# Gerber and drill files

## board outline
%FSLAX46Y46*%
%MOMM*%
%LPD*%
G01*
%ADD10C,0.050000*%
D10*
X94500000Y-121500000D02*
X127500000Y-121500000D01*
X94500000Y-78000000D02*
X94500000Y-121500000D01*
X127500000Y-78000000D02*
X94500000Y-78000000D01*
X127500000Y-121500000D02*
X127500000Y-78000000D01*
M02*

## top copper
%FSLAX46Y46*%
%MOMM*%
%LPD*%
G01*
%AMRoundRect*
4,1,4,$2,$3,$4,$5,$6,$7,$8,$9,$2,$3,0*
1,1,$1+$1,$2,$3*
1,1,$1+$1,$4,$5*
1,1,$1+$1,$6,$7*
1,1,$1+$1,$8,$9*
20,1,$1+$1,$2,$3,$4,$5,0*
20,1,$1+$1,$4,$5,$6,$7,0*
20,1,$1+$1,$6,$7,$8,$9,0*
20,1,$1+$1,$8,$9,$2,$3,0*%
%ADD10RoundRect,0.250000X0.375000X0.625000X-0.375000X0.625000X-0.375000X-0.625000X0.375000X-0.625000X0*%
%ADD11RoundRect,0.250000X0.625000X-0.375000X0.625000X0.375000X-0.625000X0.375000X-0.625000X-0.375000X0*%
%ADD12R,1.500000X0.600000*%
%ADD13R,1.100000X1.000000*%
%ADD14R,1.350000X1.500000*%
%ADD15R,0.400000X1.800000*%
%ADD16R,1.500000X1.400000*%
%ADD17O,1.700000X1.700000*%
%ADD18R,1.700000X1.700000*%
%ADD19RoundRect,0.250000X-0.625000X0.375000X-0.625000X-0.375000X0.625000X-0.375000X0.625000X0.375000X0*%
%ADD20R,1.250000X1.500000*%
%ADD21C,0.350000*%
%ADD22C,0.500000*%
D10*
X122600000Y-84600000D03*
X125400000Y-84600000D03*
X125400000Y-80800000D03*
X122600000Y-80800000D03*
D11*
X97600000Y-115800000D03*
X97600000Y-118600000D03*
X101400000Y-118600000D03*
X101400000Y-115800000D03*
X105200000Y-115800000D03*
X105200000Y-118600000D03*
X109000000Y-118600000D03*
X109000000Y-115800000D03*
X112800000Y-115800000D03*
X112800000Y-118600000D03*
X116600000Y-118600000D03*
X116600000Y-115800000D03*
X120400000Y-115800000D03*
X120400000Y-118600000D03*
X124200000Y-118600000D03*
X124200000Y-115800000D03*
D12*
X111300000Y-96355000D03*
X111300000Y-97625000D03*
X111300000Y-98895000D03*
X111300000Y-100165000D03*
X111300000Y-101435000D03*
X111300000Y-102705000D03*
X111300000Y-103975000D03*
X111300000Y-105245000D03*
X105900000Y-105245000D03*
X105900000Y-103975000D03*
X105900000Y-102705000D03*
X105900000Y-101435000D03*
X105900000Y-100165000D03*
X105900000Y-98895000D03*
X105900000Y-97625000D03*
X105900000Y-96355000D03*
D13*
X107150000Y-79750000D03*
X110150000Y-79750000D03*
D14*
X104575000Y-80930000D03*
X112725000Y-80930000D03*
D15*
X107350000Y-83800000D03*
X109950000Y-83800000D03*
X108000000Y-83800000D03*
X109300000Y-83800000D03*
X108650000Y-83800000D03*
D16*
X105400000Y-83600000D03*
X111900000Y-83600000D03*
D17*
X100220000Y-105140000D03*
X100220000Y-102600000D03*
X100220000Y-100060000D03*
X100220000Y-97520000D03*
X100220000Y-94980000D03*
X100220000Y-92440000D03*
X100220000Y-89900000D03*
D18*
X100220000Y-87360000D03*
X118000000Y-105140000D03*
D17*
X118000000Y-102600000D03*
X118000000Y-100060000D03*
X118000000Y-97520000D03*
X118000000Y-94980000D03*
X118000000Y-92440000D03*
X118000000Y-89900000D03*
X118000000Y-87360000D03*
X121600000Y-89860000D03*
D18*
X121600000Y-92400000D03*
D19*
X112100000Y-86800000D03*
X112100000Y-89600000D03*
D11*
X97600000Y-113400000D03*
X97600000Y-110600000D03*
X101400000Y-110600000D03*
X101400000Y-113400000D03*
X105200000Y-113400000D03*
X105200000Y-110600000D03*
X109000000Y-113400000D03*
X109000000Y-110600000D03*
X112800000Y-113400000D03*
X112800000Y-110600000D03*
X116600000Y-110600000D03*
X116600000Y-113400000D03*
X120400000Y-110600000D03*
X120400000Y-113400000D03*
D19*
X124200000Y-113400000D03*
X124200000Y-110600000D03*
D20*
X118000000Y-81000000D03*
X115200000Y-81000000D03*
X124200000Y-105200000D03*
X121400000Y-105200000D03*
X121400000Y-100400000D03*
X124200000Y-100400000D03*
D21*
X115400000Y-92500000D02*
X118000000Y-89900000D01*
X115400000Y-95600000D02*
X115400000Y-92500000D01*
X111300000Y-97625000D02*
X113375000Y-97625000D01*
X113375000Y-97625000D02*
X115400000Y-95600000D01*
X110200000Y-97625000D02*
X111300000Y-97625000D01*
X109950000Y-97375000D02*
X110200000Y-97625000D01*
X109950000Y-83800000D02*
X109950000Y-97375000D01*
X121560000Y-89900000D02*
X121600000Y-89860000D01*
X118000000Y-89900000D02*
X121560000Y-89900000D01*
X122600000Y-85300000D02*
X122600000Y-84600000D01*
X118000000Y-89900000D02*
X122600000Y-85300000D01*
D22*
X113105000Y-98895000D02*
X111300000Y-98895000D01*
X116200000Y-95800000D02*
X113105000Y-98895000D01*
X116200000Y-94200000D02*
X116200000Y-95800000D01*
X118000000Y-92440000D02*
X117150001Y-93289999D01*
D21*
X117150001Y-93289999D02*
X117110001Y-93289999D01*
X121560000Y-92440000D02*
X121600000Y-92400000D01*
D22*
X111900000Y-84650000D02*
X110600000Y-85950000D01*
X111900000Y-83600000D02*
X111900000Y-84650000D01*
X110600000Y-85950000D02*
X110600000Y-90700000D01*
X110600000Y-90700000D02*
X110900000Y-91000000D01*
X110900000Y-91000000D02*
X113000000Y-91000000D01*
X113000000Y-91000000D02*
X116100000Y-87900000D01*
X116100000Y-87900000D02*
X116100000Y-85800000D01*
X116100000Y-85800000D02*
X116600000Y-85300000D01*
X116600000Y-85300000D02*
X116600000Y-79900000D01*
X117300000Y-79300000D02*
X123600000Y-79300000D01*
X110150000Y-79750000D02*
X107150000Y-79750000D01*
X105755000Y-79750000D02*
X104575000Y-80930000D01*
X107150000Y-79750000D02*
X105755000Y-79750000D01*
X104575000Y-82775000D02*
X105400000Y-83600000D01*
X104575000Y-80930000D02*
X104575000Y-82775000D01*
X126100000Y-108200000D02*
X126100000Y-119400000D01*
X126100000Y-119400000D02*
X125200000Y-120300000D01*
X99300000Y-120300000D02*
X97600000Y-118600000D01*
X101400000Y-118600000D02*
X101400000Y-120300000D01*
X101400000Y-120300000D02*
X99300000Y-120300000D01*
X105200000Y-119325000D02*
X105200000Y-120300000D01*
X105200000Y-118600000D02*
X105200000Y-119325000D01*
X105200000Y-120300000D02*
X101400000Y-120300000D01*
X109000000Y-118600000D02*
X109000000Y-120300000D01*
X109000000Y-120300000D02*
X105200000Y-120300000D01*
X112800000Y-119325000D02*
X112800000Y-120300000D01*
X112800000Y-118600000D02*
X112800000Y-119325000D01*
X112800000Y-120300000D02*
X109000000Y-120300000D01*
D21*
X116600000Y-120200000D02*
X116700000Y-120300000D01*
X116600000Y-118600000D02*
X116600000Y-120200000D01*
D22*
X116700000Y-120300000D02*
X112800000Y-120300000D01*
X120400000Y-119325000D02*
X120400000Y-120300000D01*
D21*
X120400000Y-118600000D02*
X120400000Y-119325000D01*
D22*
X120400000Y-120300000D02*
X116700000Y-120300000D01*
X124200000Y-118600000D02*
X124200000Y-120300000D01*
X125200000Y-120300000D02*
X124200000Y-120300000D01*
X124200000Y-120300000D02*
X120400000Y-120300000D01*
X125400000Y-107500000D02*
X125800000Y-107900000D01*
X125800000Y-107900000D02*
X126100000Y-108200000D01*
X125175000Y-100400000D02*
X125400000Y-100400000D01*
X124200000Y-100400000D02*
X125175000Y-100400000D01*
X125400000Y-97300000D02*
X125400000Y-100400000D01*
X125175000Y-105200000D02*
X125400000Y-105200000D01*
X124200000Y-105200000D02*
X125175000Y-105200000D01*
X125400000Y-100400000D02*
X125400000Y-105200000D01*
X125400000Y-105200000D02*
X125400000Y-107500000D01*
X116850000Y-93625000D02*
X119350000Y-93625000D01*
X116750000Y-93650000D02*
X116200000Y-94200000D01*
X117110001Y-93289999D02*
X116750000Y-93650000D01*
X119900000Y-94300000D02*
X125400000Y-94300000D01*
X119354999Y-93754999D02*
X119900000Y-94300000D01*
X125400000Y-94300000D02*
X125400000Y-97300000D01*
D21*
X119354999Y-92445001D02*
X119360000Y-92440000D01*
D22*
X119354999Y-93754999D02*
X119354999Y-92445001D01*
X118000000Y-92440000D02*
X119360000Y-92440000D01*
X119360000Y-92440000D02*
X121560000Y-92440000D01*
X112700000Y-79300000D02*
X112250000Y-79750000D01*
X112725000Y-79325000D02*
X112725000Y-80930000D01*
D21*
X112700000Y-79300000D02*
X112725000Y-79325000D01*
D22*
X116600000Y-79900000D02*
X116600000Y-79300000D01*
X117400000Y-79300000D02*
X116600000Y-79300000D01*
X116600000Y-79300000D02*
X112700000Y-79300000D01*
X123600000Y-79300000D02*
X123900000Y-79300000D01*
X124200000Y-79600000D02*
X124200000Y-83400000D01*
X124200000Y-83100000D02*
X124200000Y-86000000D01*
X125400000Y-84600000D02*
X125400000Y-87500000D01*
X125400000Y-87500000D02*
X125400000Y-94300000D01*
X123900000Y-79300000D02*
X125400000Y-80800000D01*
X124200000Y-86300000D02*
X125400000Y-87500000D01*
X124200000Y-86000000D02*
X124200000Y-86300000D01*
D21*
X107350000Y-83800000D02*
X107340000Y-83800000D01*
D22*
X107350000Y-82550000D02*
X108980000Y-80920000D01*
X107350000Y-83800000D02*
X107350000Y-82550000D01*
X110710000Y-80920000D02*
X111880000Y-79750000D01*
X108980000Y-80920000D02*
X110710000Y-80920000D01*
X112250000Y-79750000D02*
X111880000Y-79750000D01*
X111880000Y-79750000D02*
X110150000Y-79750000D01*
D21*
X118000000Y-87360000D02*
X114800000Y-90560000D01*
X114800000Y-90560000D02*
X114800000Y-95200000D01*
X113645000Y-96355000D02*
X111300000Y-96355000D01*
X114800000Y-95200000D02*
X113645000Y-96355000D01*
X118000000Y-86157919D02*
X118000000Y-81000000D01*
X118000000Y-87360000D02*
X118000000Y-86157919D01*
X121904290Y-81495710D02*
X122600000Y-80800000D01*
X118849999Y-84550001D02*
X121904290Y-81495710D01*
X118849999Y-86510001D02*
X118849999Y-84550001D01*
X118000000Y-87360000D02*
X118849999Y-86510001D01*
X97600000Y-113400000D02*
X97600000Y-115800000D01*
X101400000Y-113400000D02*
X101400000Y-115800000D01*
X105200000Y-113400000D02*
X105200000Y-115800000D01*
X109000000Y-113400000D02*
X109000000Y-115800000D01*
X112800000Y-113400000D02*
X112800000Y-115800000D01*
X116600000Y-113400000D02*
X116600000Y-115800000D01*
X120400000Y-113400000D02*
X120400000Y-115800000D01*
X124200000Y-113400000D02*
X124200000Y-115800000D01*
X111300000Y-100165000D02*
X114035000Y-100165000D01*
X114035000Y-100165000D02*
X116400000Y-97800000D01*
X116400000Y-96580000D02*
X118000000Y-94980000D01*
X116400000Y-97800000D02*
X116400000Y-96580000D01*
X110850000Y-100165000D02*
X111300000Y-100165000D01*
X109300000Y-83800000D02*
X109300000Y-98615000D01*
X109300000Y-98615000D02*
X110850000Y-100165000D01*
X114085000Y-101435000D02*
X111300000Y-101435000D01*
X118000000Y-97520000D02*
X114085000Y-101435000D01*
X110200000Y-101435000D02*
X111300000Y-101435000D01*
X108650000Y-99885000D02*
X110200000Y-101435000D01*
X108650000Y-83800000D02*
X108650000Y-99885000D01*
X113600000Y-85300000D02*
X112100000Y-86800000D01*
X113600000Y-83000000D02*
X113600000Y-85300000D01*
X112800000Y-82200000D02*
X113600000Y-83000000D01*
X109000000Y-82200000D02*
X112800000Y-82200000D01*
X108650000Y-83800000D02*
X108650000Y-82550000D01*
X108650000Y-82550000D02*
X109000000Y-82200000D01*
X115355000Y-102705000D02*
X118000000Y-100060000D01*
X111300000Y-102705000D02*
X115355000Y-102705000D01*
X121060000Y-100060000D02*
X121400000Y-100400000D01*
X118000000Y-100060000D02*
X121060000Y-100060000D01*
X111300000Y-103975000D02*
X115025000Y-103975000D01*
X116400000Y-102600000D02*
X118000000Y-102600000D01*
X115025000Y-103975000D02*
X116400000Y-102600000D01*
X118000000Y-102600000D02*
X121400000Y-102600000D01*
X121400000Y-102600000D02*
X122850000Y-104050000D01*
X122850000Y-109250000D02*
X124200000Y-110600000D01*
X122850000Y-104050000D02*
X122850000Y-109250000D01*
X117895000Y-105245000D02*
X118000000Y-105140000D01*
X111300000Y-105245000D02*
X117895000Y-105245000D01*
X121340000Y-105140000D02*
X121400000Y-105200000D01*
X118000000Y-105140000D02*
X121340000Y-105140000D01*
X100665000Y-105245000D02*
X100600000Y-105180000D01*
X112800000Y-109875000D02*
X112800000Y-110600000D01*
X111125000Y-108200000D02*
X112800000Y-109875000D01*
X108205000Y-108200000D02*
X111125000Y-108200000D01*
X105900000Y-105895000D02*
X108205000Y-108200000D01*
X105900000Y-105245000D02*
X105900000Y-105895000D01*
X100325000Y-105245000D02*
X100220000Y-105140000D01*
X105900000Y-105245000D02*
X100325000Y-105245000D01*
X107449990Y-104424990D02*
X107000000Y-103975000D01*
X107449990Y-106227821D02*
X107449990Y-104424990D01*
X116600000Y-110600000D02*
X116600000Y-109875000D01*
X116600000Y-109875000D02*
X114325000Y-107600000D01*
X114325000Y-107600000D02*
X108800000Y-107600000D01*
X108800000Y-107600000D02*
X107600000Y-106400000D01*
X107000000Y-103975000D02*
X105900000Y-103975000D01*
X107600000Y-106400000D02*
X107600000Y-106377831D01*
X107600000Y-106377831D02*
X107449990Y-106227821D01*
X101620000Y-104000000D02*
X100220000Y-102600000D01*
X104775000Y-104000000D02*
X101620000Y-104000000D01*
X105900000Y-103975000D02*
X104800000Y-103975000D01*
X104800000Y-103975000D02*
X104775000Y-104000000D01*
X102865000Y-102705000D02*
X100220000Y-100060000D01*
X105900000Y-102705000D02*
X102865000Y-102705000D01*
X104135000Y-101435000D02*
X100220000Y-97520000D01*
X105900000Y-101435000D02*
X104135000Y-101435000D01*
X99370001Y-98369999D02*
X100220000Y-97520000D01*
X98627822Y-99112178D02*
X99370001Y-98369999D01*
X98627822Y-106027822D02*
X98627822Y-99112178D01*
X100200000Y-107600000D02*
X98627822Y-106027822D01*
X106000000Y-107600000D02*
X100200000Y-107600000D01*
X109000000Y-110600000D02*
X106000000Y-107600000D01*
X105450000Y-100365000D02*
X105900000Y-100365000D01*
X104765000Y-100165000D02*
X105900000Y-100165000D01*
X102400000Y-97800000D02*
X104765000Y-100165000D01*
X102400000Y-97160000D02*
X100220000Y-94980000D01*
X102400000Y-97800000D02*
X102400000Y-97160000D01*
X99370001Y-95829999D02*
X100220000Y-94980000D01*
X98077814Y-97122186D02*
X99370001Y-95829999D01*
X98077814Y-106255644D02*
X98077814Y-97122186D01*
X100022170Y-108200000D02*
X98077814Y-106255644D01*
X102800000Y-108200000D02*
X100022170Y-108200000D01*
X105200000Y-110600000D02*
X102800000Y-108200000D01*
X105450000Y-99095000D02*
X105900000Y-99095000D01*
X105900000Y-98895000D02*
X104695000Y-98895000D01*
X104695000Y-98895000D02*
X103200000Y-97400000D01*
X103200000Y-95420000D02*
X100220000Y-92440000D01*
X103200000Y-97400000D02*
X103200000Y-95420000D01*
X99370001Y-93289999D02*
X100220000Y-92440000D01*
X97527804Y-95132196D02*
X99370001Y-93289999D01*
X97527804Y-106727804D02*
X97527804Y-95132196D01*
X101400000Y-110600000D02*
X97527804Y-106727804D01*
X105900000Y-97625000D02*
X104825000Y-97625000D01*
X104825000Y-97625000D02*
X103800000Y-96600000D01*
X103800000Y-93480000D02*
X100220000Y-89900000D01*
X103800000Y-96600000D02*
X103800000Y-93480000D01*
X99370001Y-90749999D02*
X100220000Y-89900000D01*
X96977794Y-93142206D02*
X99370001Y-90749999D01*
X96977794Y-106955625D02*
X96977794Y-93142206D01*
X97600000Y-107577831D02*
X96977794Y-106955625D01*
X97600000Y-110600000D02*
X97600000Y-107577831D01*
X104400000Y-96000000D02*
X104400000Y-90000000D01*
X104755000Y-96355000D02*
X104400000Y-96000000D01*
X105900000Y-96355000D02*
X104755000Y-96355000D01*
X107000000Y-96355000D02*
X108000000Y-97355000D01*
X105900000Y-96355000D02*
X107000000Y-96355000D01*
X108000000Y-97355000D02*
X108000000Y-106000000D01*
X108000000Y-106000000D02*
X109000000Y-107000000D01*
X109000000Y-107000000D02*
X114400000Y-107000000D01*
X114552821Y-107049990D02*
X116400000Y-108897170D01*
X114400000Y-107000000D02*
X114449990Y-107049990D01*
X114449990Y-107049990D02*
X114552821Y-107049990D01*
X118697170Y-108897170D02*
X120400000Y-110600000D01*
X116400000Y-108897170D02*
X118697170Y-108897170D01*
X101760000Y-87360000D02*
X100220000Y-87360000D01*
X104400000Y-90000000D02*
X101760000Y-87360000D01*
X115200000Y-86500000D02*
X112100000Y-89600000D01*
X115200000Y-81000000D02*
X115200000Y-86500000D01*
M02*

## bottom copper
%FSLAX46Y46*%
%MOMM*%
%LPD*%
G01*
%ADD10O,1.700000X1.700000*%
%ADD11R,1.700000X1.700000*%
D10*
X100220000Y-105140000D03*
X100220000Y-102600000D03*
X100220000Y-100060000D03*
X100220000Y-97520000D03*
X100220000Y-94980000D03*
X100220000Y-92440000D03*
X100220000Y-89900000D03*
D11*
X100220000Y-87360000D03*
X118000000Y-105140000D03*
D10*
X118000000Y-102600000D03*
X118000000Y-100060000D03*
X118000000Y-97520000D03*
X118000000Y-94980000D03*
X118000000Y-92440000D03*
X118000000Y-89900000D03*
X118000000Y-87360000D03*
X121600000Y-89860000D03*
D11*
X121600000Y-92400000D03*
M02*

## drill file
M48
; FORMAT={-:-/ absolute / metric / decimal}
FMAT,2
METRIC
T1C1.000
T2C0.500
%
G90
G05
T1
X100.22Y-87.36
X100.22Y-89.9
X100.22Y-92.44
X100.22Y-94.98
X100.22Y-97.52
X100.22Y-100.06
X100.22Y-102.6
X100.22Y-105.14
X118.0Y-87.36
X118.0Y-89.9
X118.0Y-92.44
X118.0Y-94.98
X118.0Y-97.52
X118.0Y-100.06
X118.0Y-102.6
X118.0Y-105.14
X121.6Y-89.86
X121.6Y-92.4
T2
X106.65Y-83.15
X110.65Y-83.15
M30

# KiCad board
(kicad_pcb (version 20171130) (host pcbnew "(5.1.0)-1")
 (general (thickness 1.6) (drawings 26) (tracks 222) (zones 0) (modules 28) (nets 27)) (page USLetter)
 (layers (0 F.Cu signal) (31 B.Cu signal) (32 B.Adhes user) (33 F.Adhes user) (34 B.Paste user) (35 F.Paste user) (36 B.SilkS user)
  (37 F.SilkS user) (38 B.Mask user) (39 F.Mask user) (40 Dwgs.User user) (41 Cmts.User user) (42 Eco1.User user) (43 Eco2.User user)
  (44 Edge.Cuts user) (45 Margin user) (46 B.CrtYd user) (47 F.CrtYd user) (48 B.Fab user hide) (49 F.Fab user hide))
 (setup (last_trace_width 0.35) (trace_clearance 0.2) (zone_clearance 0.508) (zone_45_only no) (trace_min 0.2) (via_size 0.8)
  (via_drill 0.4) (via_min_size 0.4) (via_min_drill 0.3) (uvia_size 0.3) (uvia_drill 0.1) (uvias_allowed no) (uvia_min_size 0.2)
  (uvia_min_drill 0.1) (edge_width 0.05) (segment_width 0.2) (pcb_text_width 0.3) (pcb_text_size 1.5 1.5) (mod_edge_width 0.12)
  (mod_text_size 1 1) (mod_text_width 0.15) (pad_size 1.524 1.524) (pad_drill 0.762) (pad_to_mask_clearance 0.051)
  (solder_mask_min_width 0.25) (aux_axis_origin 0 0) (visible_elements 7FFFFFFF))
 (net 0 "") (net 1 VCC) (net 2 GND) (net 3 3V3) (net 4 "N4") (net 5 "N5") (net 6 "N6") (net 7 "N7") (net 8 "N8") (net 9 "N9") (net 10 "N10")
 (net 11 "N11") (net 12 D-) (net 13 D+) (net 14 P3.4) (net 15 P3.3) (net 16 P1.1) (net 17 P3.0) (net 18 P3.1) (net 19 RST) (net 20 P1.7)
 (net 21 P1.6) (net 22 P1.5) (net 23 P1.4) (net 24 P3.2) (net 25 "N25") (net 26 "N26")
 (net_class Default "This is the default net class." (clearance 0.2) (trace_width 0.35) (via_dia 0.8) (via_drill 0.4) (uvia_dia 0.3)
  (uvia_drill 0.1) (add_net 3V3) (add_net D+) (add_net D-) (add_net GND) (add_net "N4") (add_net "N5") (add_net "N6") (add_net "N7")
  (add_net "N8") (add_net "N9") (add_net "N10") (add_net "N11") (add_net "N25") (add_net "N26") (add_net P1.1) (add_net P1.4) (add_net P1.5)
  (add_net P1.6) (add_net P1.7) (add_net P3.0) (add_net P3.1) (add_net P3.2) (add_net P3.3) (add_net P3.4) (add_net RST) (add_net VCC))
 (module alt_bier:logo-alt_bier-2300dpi (layer F.Cu) (at 106.36 90.52)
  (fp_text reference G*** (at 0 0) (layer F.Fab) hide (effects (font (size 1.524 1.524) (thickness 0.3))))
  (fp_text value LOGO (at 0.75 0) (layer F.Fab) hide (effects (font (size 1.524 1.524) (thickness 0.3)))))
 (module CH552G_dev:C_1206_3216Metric (layer F.Cu) (at 124 84.6 180)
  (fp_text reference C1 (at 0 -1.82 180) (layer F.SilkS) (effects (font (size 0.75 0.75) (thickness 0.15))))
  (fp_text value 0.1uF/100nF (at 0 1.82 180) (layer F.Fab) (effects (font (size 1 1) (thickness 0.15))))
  (pad 2 smd roundrect (at 1.4 0 180) (size 1.25 1.75) (layers F.Cu F.Paste F.Mask) (roundrect_rratio 0.2) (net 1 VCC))
  (pad 1 smd roundrect (at -1.4 0 180) (size 1.25 1.75) (layers F.Cu F.Paste F.Mask) (roundrect_rratio 0.2) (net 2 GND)))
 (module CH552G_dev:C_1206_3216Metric (layer F.Cu) (at 124 80.8 180)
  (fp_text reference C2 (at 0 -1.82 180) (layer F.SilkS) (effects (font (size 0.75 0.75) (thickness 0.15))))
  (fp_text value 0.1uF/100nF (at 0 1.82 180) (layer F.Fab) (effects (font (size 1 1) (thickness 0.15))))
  (pad 1 smd roundrect (at -1.4 0 180) (size 1.25 1.75) (layers F.Cu F.Paste F.Mask) (roundrect_rratio 0.2) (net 2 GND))
  (pad 2 smd roundrect (at 1.4 0 180) (size 1.25 1.75) (layers F.Cu F.Paste F.Mask) (roundrect_rratio 0.2) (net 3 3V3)))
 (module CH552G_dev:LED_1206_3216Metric (layer F.Cu) (at 97.6 117.2 90)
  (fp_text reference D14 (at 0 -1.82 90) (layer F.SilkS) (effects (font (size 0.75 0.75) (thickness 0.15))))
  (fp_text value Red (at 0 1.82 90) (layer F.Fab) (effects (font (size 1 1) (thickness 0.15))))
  (pad 2 smd roundrect (at 1.4 0 90) (size 1.25 1.75) (layers F.Cu F.Paste F.Mask) (roundrect_rratio 0.2) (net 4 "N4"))
  (pad 1 smd roundrect (at -1.4 0 90) (size 1.25 1.75) (layers F.Cu F.Paste F.Mask) (roundrect_rratio 0.2) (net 2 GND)))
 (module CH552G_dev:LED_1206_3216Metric (layer F.Cu) (at 101.4 117.2 90)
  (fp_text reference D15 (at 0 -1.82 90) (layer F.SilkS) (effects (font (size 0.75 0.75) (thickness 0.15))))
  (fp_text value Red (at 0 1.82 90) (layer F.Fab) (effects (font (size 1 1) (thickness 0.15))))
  (pad 1 smd roundrect (at -1.4 0 90) (size 1.25 1.75) (layers F.Cu F.Paste F.Mask) (roundrect_rratio 0.2) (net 2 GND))
  (pad 2 smd roundrect (at 1.4 0 90) (size 1.25 1.75) (layers F.Cu F.Paste F.Mask) (roundrect_rratio 0.2) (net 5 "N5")))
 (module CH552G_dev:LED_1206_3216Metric (layer F.Cu) (at 105.2 117.2 90)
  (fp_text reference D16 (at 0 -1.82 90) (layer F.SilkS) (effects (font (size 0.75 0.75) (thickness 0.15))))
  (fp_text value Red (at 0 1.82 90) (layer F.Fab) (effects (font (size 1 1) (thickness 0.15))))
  (pad 2 smd roundrect (at 1.4 0 90) (size 1.25 1.75) (layers F.Cu F.Paste F.Mask) (roundrect_rratio 0.2) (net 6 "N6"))
  (pad 1 smd roundrect (at -1.4 0 90) (size 1.25 1.75) (layers F.Cu F.Paste F.Mask) (roundrect_rratio 0.2) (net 2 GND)))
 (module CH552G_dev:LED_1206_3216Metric (layer F.Cu) (at 109 117.2 90)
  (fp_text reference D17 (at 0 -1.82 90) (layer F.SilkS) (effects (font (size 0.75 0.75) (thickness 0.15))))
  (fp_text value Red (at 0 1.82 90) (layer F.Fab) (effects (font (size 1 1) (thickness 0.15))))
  (pad 1 smd roundrect (at -1.4 0 90) (size 1.25 1.75) (layers F.Cu F.Paste F.Mask) (roundrect_rratio 0.2) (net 2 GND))
  (pad 2 smd roundrect (at 1.4 0 90) (size 1.25 1.75) (layers F.Cu F.Paste F.Mask) (roundrect_rratio 0.2) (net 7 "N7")))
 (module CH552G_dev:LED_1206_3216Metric (layer F.Cu) (at 112.8 117.2 90)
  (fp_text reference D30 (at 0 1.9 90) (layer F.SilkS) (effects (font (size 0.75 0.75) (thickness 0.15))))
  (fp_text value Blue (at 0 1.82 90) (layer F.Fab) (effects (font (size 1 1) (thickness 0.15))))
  (pad 2 smd roundrect (at 1.4 0 90) (size 1.25 1.75) (layers F.Cu F.Paste F.Mask) (roundrect_rratio 0.2) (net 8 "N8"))
  (pad 1 smd roundrect (at -1.4 0 90) (size 1.25 1.75) (layers F.Cu F.Paste F.Mask) (roundrect_rratio 0.2) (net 2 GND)))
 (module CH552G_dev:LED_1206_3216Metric (layer F.Cu) (at 116.6 117.2 90)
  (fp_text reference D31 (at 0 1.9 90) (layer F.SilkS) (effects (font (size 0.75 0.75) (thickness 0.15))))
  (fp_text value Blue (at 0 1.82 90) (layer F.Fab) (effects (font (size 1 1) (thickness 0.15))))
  (pad 1 smd roundrect (at -1.4 0 90) (size 1.25 1.75) (layers F.Cu F.Paste F.Mask) (roundrect_rratio 0.2) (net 2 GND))
  (pad 2 smd roundrect (at 1.4 0 90) (size 1.25 1.75) (layers F.Cu F.Paste F.Mask) (roundrect_rratio 0.2) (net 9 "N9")))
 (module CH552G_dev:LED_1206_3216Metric (layer F.Cu) (at 120.4 117.2 90)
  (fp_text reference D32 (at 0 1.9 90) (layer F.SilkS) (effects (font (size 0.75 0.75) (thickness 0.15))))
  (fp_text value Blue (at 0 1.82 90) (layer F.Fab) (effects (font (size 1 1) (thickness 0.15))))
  (pad 2 smd roundrect (at 1.4 0 90) (size 1.25 1.75) (layers F.Cu F.Paste F.Mask) (roundrect_rratio 0.2) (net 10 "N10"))
  (pad 1 smd roundrect (at -1.4 0 90) (size 1.25 1.75) (layers F.Cu F.Paste F.Mask) (roundrect_rratio 0.2) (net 2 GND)))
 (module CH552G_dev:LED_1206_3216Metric (layer F.Cu) (at 124.2 117.2 90)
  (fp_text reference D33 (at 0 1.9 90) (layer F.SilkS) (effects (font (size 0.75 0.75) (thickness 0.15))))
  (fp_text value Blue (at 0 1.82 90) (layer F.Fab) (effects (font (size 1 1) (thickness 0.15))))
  (pad 1 smd roundrect (at -1.4 0 90) (size 1.25 1.75) (layers F.Cu F.Paste F.Mask) (roundrect_rratio 0.2) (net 2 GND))
  (pad 2 smd roundrect (at 1.4 0 90) (size 1.25 1.75) (layers F.Cu F.Paste F.Mask) (roundrect_rratio 0.2) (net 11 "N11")))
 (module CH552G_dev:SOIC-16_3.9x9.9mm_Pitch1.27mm (layer F.Cu) (at 108.6 100.8)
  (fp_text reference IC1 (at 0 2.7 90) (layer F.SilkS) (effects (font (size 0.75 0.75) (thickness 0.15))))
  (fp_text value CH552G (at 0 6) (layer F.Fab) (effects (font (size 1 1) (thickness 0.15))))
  (pad 16 smd rect (at 2.7 -4.445) (size 1.5 0.6) (layers F.Cu F.Paste F.Mask) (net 3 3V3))
  (pad 15 smd rect (at 2.7 -3.175) (size 1.5 0.6) (layers F.Cu F.Paste F.Mask) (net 1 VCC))
  (pad 14 smd rect (at 2.7 -1.905) (size 1.5 0.6) (layers F.Cu F.Paste F.Mask) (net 2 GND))
  (pad 13 smd rect (at 2.7 -0.635) (size 1.5 0.6) (layers F.Cu F.Paste F.Mask) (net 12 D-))
  (pad 12 smd rect (at 2.7 0.635) (size 1.5 0.6) (layers F.Cu F.Paste F.Mask) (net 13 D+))
  (pad 11 smd rect (at 2.7 1.905) (size 1.5 0.6) (layers F.Cu F.Paste F.Mask) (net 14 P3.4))
  (pad 10 smd rect (at 2.7 3.175) (size 1.5 0.6) (layers F.Cu F.Paste F.Mask) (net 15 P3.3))
  (pad 9 smd rect (at 2.7 4.445) (size 1.5 0.6) (layers F.Cu F.Paste F.Mask) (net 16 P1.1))
  (pad 8 smd rect (at -2.7 4.445) (size 1.5 0.6) (layers F.Cu F.Paste F.Mask) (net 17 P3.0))
  (pad 7 smd rect (at -2.7 3.175) (size 1.5 0.6) (layers F.Cu F.Paste F.Mask) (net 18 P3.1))
  (pad 6 smd rect (at -2.7 1.905) (size 1.5 0.6) (layers F.Cu F.Paste F.Mask) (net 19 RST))
  (pad 5 smd rect (at -2.7 0.635) (size 1.5 0.6) (layers F.Cu F.Paste F.Mask) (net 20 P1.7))
  (pad 4 smd rect (at -2.7 -0.635) (size 1.5 0.6) (layers F.Cu F.Paste F.Mask) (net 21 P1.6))
  (pad 3 smd rect (at -2.7 -1.905) (size 1.5 0.6) (layers F.Cu F.Paste F.Mask) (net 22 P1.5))
  (pad 2 smd rect (at -2.7 -3.175) (size 1.5 0.6) (layers F.Cu F.Paste F.Mask) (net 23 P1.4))
  (pad 1 smd rect (at -2.7 -4.445) (size 1.5 0.6) (layers F.Cu F.Paste F.Mask) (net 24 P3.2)))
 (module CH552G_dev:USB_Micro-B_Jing (layer F.Cu) (at 108.65 81.7 180)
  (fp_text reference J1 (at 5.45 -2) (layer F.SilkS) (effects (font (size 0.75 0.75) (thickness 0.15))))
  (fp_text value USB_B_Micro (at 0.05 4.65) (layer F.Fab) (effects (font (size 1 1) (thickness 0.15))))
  (pad 6 smd rect (at 1.5 1.95 180) (size 1.1 1) (layers F.Cu F.Paste F.Mask) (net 2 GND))
  (pad 6 smd rect (at -1.5 1.95 180) (size 1.1 1) (layers F.Cu F.Paste F.Mask) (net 2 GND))
  (pad 6 smd rect (at 4.075 0.77 180) (size 1.35 1.5) (layers F.Cu F.Paste F.Mask) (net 2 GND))
  (pad 6 smd rect (at -4.075 0.77 180) (size 1.35 1.5) (layers F.Cu F.Paste F.Mask) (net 2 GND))
  (pad "" np_thru_hole circle (at 2 -1.45 180) (size 0.5 0.5) (drill 0.5) (layers *.Cu *.Mask))
  (pad "" np_thru_hole circle (at -2 -1.45 180) (size 0.5 0.5) (drill 0.5) (layers *.Cu *.Mask))
  (pad 5 smd rect (at 1.3 -2.1 180) (size 0.4 1.8) (layers F.Cu F.Paste F.Mask) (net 2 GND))
  (pad 1 smd rect (at -1.3 -2.1 180) (size 0.4 1.8) (layers F.Cu F.Paste F.Mask) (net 1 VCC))
  (pad 4 smd rect (at 0.65 -2.1 180) (size 0.4 1.8) (layers F.Cu F.Paste F.Mask) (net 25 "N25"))
  (pad 2 smd rect (at -0.65 -2.1 180) (size 0.4 1.8) (layers F.Cu F.Paste F.Mask) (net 12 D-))
  (pad 3 smd rect (at 0 -2.1 180) (size 0.4 1.8) (layers F.Cu F.Paste F.Mask) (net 13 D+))
  (pad 6 smd rect (at 3.25 -1.9 180) (size 1.5 1.4) (layers F.Cu F.Paste F.Mask) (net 2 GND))
  (pad 6 smd rect (at -3.25 -1.9 180) (size 1.5 1.4) (layers F.Cu F.Paste F.Mask) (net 2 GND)))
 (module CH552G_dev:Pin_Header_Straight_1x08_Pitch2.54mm (layer F.Cu) (at 100.22 87.36)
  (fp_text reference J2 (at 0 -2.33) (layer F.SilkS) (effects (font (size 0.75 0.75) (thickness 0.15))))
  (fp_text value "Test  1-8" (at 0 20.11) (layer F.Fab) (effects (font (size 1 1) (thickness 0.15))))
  (pad 8 thru_hole oval (at 0 17.78) (size 1.7 1.7) (drill 1) (layers *.Cu *.Mask) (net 17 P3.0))
  (pad 7 thru_hole oval (at 0 15.24) (size 1.7 1.7) (drill 1) (layers *.Cu *.Mask) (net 18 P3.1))
  (pad 6 thru_hole oval (at 0 12.7) (size 1.7 1.7) (drill 1) (layers *.Cu *.Mask) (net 19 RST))
  (pad 5 thru_hole oval (at 0 10.16) (size 1.7 1.7) (drill 1) (layers *.Cu *.Mask) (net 20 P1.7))
  (pad 4 thru_hole oval (at 0 7.62) (size 1.7 1.7) (drill 1) (layers *.Cu *.Mask) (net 21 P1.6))
  (pad 3 thru_hole oval (at 0 5.08) (size 1.7 1.7) (drill 1) (layers *.Cu *.Mask) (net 22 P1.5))
  (pad 2 thru_hole oval (at 0 2.54) (size 1.7 1.7) (drill 1) (layers *.Cu *.Mask) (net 23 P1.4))
  (pad 1 thru_hole rect (at 0 0) (size 1.7 1.7) (drill 1) (layers *.Cu *.Mask) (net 24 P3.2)))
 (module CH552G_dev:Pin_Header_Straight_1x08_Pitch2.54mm (layer F.Cu) (at 118 105.14 180)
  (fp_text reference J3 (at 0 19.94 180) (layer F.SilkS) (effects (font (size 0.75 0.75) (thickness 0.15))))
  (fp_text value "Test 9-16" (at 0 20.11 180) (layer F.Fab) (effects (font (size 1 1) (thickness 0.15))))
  (pad 1 thru_hole rect (at 0 0 180) (size 1.7 1.7) (drill 1) (layers *.Cu *.Mask) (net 16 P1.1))
  (pad 2 thru_hole oval (at 0 2.54 180) (size 1.7 1.7) (drill 1) (layers *.Cu *.Mask) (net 15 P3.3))
  (pad 3 thru_hole oval (at 0 5.08 180) (size 1.7 1.7) (drill 1) (layers *.Cu *.Mask) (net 14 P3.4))
  (pad 4 thru_hole oval (at 0 7.62 180) (size 1.7 1.7) (drill 1) (layers *.Cu *.Mask) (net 13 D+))
  (pad 5 thru_hole oval (at 0 10.16 180) (size 1.7 1.7) (drill 1) (layers *.Cu *.Mask) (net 12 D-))
  (pad 6 thru_hole oval (at 0 12.7 180) (size 1.7 1.7) (drill 1) (layers *.Cu *.Mask) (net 2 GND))
  (pad 7 thru_hole oval (at 0 15.24 180) (size 1.7 1.7) (drill 1) (layers *.Cu *.Mask) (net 1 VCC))
  (pad 8 thru_hole oval (at 0 17.78 180) (size 1.7 1.7) (drill 1) (layers *.Cu *.Mask) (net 3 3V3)))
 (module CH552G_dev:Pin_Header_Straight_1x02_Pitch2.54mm (layer F.Cu) (at 121.6 92.4 180)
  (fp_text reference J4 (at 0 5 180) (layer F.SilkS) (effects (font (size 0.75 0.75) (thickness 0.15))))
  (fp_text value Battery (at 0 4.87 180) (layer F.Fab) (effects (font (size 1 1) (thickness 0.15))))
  (pad 2 thru_hole oval (at 0 2.54 180) (size 1.7 1.7) (drill 1) (layers *.Cu *.Mask) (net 1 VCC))
  (pad 1 thru_hole rect (at 0 0 180) (size 1.7 1.7) (drill 1) (layers *.Cu *.Mask) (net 2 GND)))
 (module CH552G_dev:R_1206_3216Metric (layer F.Cu) (at 112.1 88.2 270)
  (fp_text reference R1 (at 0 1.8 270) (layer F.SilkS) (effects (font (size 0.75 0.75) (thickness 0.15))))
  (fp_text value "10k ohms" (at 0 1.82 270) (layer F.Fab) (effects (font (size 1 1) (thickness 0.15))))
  (pad 1 smd roundrect (at -1.4 0 270) (size 1.25 1.75) (layers F.Cu F.Paste F.Mask) (roundrect_rratio 0.2) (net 13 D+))
  (pad 2 smd roundrect (at 1.4 0 270) (size 1.25 1.75) (layers F.Cu F.Paste F.Mask) (roundrect_rratio 0.2) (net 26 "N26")))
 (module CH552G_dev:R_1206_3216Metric (layer F.Cu) (at 97.6 112 90)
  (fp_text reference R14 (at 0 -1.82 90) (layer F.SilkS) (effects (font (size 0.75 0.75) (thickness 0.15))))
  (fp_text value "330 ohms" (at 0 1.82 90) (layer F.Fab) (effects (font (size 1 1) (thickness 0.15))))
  (pad 1 smd roundrect (at -1.4 0 90) (size 1.25 1.75) (layers F.Cu F.Paste F.Mask) (roundrect_rratio 0.2) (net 4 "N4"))
  (pad 2 smd roundrect (at 1.4 0 90) (size 1.25 1.75) (layers F.Cu F.Paste F.Mask) (roundrect_rratio 0.2) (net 23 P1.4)))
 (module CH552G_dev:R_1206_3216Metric (layer F.Cu) (at 101.4 112 90)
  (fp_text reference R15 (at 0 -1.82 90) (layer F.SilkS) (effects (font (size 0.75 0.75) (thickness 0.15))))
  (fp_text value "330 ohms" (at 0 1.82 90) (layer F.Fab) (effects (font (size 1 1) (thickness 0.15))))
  (pad 2 smd roundrect (at 1.4 0 90) (size 1.25 1.75) (layers F.Cu F.Paste F.Mask) (roundrect_rratio 0.2) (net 22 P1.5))
  (pad 1 smd roundrect (at -1.4 0 90) (size 1.25 1.75) (layers F.Cu F.Paste F.Mask) (roundrect_rratio 0.2) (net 5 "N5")))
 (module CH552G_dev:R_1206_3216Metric (layer F.Cu) (at 105.2 112 90)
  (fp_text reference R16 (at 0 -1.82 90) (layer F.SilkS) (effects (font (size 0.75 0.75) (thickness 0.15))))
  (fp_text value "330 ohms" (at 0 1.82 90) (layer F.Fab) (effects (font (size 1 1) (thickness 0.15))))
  (pad 1 smd roundrect (at -1.4 0 90) (size 1.25 1.75) (layers F.Cu F.Paste F.Mask) (roundrect_rratio 0.2) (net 6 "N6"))
  (pad 2 smd roundrect (at 1.4 0 90) (size 1.25 1.75) (layers F.Cu F.Paste F.Mask) (roundrect_rratio 0.2) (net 21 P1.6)))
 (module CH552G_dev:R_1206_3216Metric (layer F.Cu) (at 109 112 90)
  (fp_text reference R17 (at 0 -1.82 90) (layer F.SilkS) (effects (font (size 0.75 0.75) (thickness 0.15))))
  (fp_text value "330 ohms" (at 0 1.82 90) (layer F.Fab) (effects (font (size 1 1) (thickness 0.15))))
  (pad 1 smd roundrect (at -1.4 0 90) (size 1.25 1.75) (layers F.Cu F.Paste F.Mask) (roundrect_rratio 0.2) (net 7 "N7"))
  (pad 2 smd roundrect (at 1.4 0 90) (size 1.25 1.75) (layers F.Cu F.Paste F.Mask) (roundrect_rratio 0.2) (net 20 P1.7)))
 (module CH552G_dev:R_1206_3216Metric (layer F.Cu) (at 112.8 112 90)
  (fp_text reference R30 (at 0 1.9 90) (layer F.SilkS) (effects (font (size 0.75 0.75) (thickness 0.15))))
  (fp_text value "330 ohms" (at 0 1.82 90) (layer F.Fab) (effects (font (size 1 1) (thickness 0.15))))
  (pad 1 smd roundrect (at -1.4 0 90) (size 1.25 1.75) (layers F.Cu F.Paste F.Mask) (roundrect_rratio 0.2) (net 8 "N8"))
  (pad 2 smd roundrect (at 1.4 0 90) (size 1.25 1.75) (layers F.Cu F.Paste F.Mask) (roundrect_rratio 0.2) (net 17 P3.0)))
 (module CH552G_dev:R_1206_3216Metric (layer F.Cu) (at 116.6 112 90)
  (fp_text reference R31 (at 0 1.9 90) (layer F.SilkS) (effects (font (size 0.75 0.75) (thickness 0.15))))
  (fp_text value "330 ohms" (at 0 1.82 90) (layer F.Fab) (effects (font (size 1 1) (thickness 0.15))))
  (pad 2 smd roundrect (at 1.4 0 90) (size 1.25 1.75) (layers F.Cu F.Paste F.Mask) (roundrect_rratio 0.2) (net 18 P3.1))
  (pad 1 smd roundrect (at -1.4 0 90) (size 1.25 1.75) (layers F.Cu F.Paste F.Mask) (roundrect_rratio 0.2) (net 9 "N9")))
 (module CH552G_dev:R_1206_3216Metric (layer F.Cu) (at 120.4 112 90)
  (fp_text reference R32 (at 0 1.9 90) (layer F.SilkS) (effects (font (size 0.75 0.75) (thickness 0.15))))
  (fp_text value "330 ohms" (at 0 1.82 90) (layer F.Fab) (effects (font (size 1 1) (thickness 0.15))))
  (pad 2 smd roundrect (at 1.4 0 90) (size 1.25 1.75) (layers F.Cu F.Paste F.Mask) (roundrect_rratio 0.2) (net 24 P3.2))
  (pad 1 smd roundrect (at -1.4 0 90) (size 1.25 1.75) (layers F.Cu F.Paste F.Mask) (roundrect_rratio 0.2) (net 10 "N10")))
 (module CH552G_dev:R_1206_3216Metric (layer F.Cu) (at 124.2 112 270)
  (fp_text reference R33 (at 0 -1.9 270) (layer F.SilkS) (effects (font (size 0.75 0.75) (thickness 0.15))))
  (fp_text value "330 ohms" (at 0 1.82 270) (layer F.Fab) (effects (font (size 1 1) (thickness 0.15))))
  (pad 2 smd roundrect (at 1.4 0 270) (size 1.25 1.75) (layers F.Cu F.Paste F.Mask) (roundrect_rratio 0.2) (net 11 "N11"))
  (pad 1 smd roundrect (at -1.4 0 270) (size 1.25 1.75) (layers F.Cu F.Paste F.Mask) (roundrect_rratio 0.2) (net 15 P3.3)))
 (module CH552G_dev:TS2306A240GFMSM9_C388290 (layer F.Cu) (at 116.6 81 180)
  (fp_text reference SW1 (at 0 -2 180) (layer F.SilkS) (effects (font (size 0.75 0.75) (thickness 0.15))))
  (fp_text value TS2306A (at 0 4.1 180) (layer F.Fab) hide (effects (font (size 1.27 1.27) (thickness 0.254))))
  (pad 1 smd rect (at -1.4 0 180) (size 1.25 1.5) (layers F.Cu F.Paste F.Mask) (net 3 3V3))
  (pad 2 smd rect (at 1.4 0 180) (size 1.25 1.5) (layers F.Cu F.Paste F.Mask) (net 26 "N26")))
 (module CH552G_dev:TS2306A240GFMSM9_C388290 (layer F.Cu) (at 122.8 105.2)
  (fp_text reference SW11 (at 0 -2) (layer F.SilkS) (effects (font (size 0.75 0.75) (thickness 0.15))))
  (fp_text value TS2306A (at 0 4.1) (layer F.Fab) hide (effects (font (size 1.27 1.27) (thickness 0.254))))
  (pad 2 smd rect (at 1.4 0) (size 1.25 1.5) (layers F.Cu F.Paste F.Mask) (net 2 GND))
  (pad 1 smd rect (at -1.4 0) (size 1.25 1.5) (layers F.Cu F.Paste F.Mask) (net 16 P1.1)))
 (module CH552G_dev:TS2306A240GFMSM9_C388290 (layer F.Cu) (at 122.8 100.4)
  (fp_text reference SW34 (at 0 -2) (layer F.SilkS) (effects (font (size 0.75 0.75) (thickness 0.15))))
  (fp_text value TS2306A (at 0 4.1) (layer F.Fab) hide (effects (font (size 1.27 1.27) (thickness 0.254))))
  (pad 1 smd rect (at -1.4 0) (size 1.25 1.5) (layers F.Cu F.Paste F.Mask) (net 14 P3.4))
  (pad 2 smd rect (at 1.4 0) (size 1.25 1.5) (layers F.Cu F.Paste F.Mask) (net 2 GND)))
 (gr_line (start 94.5 121.5) (end 127.5 121.5) (layer Edge.Cuts) (width 0.05))
 (gr_line (start 94.5 78) (end 94.5 121.5) (layer Edge.Cuts) (width 0.05))
 (gr_line (start 127.5 78) (end 94.5 78) (layer Edge.Cuts) (width 0.05))
 (gr_line (start 127.5 121.5) (end 127.5 78) (layer Edge.Cuts) (width 0.05))
 (segment (start 115.4 92.5) (end 118 89.9) (width 0.35) (layer F.Cu) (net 1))
 (segment (start 115.4 95.6) (end 115.4 92.5) (width 0.35) (layer F.Cu) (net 1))
 (segment (start 111.3 97.625) (end 113.375 97.625) (width 0.35) (layer F.Cu) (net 1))
 (segment (start 113.375 97.625) (end 115.4 95.6) (width 0.35) (layer F.Cu) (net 1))
 (segment (start 110.2 97.625) (end 111.3 97.625) (width 0.35) (layer F.Cu) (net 1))
 (segment (start 109.95 97.375) (end 110.2 97.625) (width 0.35) (layer F.Cu) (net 1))
 (segment (start 109.95 83.8) (end 109.95 97.375) (width 0.35) (layer F.Cu) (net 1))
 (segment (start 121.56 89.9) (end 121.6 89.86) (width 0.35) (layer F.Cu) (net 1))
 (segment (start 118 89.9) (end 121.56 89.9) (width 0.35) (layer F.Cu) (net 1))
 (segment (start 122.6 85.3) (end 122.6 84.6) (width 0.35) (layer F.Cu) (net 1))
 (segment (start 118 89.9) (end 122.6 85.3) (width 0.35) (layer F.Cu) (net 1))
 (segment (start 113.105 98.895) (end 111.3 98.895) (width 0.5) (layer F.Cu) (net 2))
 (segment (start 116.2 95.8) (end 113.105 98.895) (width 0.5) (layer F.Cu) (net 2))
 (segment (start 116.2 94.2) (end 116.2 95.8) (width 0.5) (layer F.Cu) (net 2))
 (segment (start 118 92.44) (end 117.150001 93.289999) (width 0.5) (layer F.Cu) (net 2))
 (segment (start 117.150001 93.289999) (end 117.110001 93.289999) (width 0.35) (layer F.Cu) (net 2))
 (segment (start 121.56 92.44) (end 121.6 92.4) (width 0.35) (layer F.Cu) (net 2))
 (segment (start 111.9 84.65) (end 110.6 85.95) (width 0.5) (layer F.Cu) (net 2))
 (segment (start 111.9 83.6) (end 111.9 84.65) (width 0.5) (layer F.Cu) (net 2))
 (segment (start 110.6 85.95) (end 110.6 90.7) (width 0.5) (layer F.Cu) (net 2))
 (segment (start 110.6 90.7) (end 110.9 91) (width 0.5) (layer F.Cu) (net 2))
 (segment (start 110.9 91) (end 113 91) (width 0.5) (layer F.Cu) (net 2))
 (segment (start 113 91) (end 116.1 87.9) (width 0.5) (layer F.Cu) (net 2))
 (segment (start 116.1 87.9) (end 116.1 85.8) (width 0.5) (layer F.Cu) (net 2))
 (segment (start 116.1 85.8) (end 116.6 85.3) (width 0.5) (layer F.Cu) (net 2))
 (segment (start 116.6 85.3) (end 116.6 79.9) (width 0.5) (layer F.Cu) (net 2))
 (segment (start 117.3 79.3) (end 123.6 79.3) (width 0.5) (layer F.Cu) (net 2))
 (segment (start 110.15 79.75) (end 107.15 79.75) (width 0.5) (layer F.Cu) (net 2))
 (segment (start 105.755 79.75) (end 104.575 80.93) (width 0.5) (layer F.Cu) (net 2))
 (segment (start 107.15 79.75) (end 105.755 79.75) (width 0.5) (layer F.Cu) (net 2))
 (segment (start 104.575 82.775) (end 105.4 83.6) (width 0.5) (layer F.Cu) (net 2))
 (segment (start 104.575 80.93) (end 104.575 82.775) (width 0.5) (layer F.Cu) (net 2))
 (segment (start 126.1 108.2) (end 126.1 119.4) (width 0.5) (layer F.Cu) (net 2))
 (segment (start 126.1 119.4) (end 125.2 120.3) (width 0.5) (layer F.Cu) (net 2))
 (segment (start 99.3 120.3) (end 97.6 118.6) (width 0.5) (layer F.Cu) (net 2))
 (segment (start 101.4 118.6) (end 101.4 120.3) (width 0.5) (layer F.Cu) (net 2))
 (segment (start 101.4 120.3) (end 99.3 120.3) (width 0.5) (layer F.Cu) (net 2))
 (segment (start 105.2 119.325) (end 105.2 120.3) (width 0.5) (layer F.Cu) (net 2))
 (segment (start 105.2 118.6) (end 105.2 119.325) (width 0.5) (layer F.Cu) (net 2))
 (segment (start 105.2 120.3) (end 101.4 120.3) (width 0.5) (layer F.Cu) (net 2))
 (segment (start 109 118.6) (end 109 120.3) (width 0.5) (layer F.Cu) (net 2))
 (segment (start 109 120.3) (end 105.2 120.3) (width 0.5) (layer F.Cu) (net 2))
 (segment (start 112.8 119.325) (end 112.8 120.3) (width 0.5) (layer F.Cu) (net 2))
 (segment (start 112.8 118.6) (end 112.8 119.325) (width 0.5) (layer F.Cu) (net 2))
 (segment (start 112.8 120.3) (end 109 120.3) (width 0.5) (layer F.Cu) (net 2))
 (segment (start 116.6 120.2) (end 116.7 120.3) (width 0.35) (layer F.Cu) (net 2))
 (segment (start 116.6 118.6) (end 116.6 120.2) (width 0.35) (layer F.Cu) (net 2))
 (segment (start 116.7 120.3) (end 112.8 120.3) (width 0.5) (layer F.Cu) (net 2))
 (segment (start 120.4 119.325) (end 120.4 120.3) (width 0.5) (layer F.Cu) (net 2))
 (segment (start 120.4 118.6) (end 120.4 119.325) (width 0.35) (layer F.Cu) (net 2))
 (segment (start 120.4 120.3) (end 116.7 120.3) (width 0.5) (layer F.Cu) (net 2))
 (segment (start 124.2 118.6) (end 124.2 120.3) (width 0.5) (layer F.Cu) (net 2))
 (segment (start 125.2 120.3) (end 124.2 120.3) (width 0.5) (layer F.Cu) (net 2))
 (segment (start 124.2 120.3) (end 120.4 120.3) (width 0.5) (layer F.Cu) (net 2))
 (segment (start 125.4 107.5) (end 125.8 107.9) (width 0.5) (layer F.Cu) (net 2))
 (segment (start 125.8 107.9) (end 126.1 108.2) (width 0.5) (layer F.Cu) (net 2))
 (segment (start 125.175 100.4) (end 125.4 100.4) (width 0.5) (layer F.Cu) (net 2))
 (segment (start 124.2 100.4) (end 125.175 100.4) (width 0.5) (layer F.Cu) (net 2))
 (segment (start 125.4 97.3) (end 125.4 100.4) (width 0.5) (layer F.Cu) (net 2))
 (segment (start 125.175 105.2) (end 125.4 105.2) (width 0.5) (layer F.Cu) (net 2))
 (segment (start 124.2 105.2) (end 125.175 105.2) (width 0.5) (layer F.Cu) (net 2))
 (segment (start 125.4 100.4) (end 125.4 105.2) (width 0.5) (layer F.Cu) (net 2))
 (segment (start 125.4 105.2) (end 125.4 107.5) (width 0.5) (layer F.Cu) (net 2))
 (segment (start 116.85 93.625) (end 119.35 93.625) (width 0.5) (layer F.Cu) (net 2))
 (segment (start 116.75 93.65) (end 116.2 94.2) (width 0.5) (layer F.Cu) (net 2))
 (segment (start 117.110001 93.289999) (end 116.75 93.65) (width 0.5) (layer F.Cu) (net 2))
 (segment (start 119.9 94.3) (end 125.4 94.3) (width 0.5) (layer F.Cu) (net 2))
 (segment (start 119.354999 93.754999) (end 119.9 94.3) (width 0.5) (layer F.Cu) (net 2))
 (segment (start 125.4 94.3) (end 125.4 97.3) (width 0.5) (layer F.Cu) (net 2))
 (segment (start 119.354999 92.445001) (end 119.36 92.44) (width 0.35) (layer F.Cu) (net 2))
 (segment (start 119.354999 93.754999) (end 119.354999 92.445001) (width 0.5) (layer F.Cu) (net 2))
 (segment (start 118 92.44) (end 119.36 92.44) (width 0.5) (layer F.Cu) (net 2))
 (segment (start 119.36 92.44) (end 121.56 92.44) (width 0.5) (layer F.Cu) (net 2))
 (segment (start 112.7 79.3) (end 112.25 79.75) (width 0.5) (layer F.Cu) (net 2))
 (segment (start 112.725 79.325) (end 112.725 80.93) (width 0.5) (layer F.Cu) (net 2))
 (segment (start 112.7 79.3) (end 112.725 79.325) (width 0.35) (layer F.Cu) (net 2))
 (segment (start 116.6 79.9) (end 116.6 79.3) (width 0.5) (layer F.Cu) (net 2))
 (segment (start 117.4 79.3) (end 116.6 79.3) (width 0.5) (layer F.Cu) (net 2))
 (segment (start 116.6 79.3) (end 112.7 79.3) (width 0.5) (layer F.Cu) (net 2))
 (segment (start 123.6 79.3) (end 123.9 79.3) (width 0.5) (layer F.Cu) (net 2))
 (segment (start 124.2 79.6) (end 124.2 83.4) (width 0.5) (layer F.Cu) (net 2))
 (segment (start 124.2 83.1) (end 124.2 86) (width 0.5) (layer F.Cu) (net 2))
 (segment (start 125.4 84.6) (end 125.4 87.5) (width 0.5) (layer F.Cu) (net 2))
 (segment (start 125.4 87.5) (end 125.4 94.3) (width 0.5) (layer F.Cu) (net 2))
 (segment (start 123.9 79.3) (end 125.4 80.8) (width 0.5) (layer F.Cu) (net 2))
 (segment (start 124.2 86.3) (end 125.4 87.5) (width 0.5) (layer F.Cu) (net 2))
 (segment (start 124.2 86) (end 124.2 86.3) (width 0.5) (layer F.Cu) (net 2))
 (segment (start 107.35 83.8) (end 107.34 83.8) (width 0.35) (layer F.Cu) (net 2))
 (segment (start 107.35 82.55) (end 108.98 80.92) (width 0.5) (layer F.Cu) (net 2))
 (segment (start 107.35 83.8) (end 107.35 82.55) (width 0.5) (layer F.Cu) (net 2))
 (segment (start 110.71 80.92) (end 111.88 79.75) (width 0.5) (layer F.Cu) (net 2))
 (segment (start 108.98 80.92) (end 110.71 80.92) (width 0.5) (layer F.Cu) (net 2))
 (segment (start 112.25 79.75) (end 111.88 79.75) (width 0.5) (layer F.Cu) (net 2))
 (segment (start 111.88 79.75) (end 110.15 79.75) (width 0.5) (layer F.Cu) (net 2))
 (segment (start 118 87.36) (end 114.8 90.56) (width 0.35) (layer F.Cu) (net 3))
 (segment (start 114.8 90.56) (end 114.8 95.2) (width 0.35) (layer F.Cu) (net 3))
 (segment (start 113.645 96.355) (end 111.3 96.355) (width 0.35) (layer F.Cu) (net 3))
 (segment (start 114.8 95.2) (end 113.645 96.355) (width 0.35) (layer F.Cu) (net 3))
 (segment (start 118 86.157919) (end 118 81) (width 0.35) (layer F.Cu) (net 3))
 (segment (start 118 87.36) (end 118 86.157919) (width 0.35) (layer F.Cu) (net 3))
 (segment (start 121.90429 81.49571) (end 122.6 80.8) (width 0.35) (layer F.Cu) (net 3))
 (segment (start 118.849999 84.550001) (end 121.90429 81.49571) (width 0.35) (layer F.Cu) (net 3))
 (segment (start 118.849999 86.510001) (end 118.849999 84.550001) (width 0.35) (layer F.Cu) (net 3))
 (segment (start 118 87.36) (end 118.849999 86.510001) (width 0.35) (layer F.Cu) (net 3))
 (segment (start 97.6 113.4) (end 97.6 115.8) (width 0.35) (layer F.Cu) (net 4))
 (segment (start 101.4 113.4) (end 101.4 115.8) (width 0.35) (layer F.Cu) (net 5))
 (segment (start 105.2 113.4) (end 105.2 115.8) (width 0.35) (layer F.Cu) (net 6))
 (segment (start 109 113.4) (end 109 115.8) (width 0.35) (layer F.Cu) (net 7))
 (segment (start 112.8 113.4) (end 112.8 115.8) (width 0.35) (layer F.Cu) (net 8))
 (segment (start 116.6 113.4) (end 116.6 115.8) (width 0.35) (layer F.Cu) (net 9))
 (segment (start 120.4 113.4) (end 120.4 115.8) (width 0.35) (layer F.Cu) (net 10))
 (segment (start 124.2 113.4) (end 124.2 115.8) (width 0.35) (layer F.Cu) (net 11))
 (segment (start 111.3 100.165) (end 114.035 100.165) (width 0.35) (layer F.Cu) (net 12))
 (segment (start 114.035 100.165) (end 116.4 97.8) (width 0.35) (layer F.Cu) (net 12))
 (segment (start 116.4 96.58) (end 118 94.98) (width 0.35) (layer F.Cu) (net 12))
 (segment (start 116.4 97.8) (end 116.4 96.58) (width 0.35) (layer F.Cu) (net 12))
 (segment (start 110.85 100.165) (end 111.3 100.165) (width 0.35) (layer F.Cu) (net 12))
 (segment (start 109.3 83.8) (end 109.3 98.615) (width 0.35) (layer F.Cu) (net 12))
 (segment (start 109.3 98.615) (end 110.85 100.165) (width 0.35) (layer F.Cu) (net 12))
 (segment (start 114.085 101.435) (end 111.3 101.435) (width 0.35) (layer F.Cu) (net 13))
 (segment (start 118 97.52) (end 114.085 101.435) (width 0.35) (layer F.Cu) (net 13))
 (segment (start 110.2 101.435) (end 111.3 101.435) (width 0.35) (layer F.Cu) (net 13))
 (segment (start 108.65 99.885) (end 110.2 101.435) (width 0.35) (layer F.Cu) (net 13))
 (segment (start 108.65 83.8) (end 108.65 99.885) (width 0.35) (layer F.Cu) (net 13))
 (segment (start 113.6 85.3) (end 112.1 86.8) (width 0.35) (layer F.Cu) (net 13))
 (segment (start 113.6 83) (end 113.6 85.3) (width 0.35) (layer F.Cu) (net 13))
 (segment (start 112.8 82.2) (end 113.6 83) (width 0.35) (layer F.Cu) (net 13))
 (segment (start 109 82.2) (end 112.8 82.2) (width 0.35) (layer F.Cu) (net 13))
 (segment (start 108.65 83.8) (end 108.65 82.55) (width 0.35) (layer F.Cu) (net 13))
 (segment (start 108.65 82.55) (end 109 82.2) (width 0.35) (layer F.Cu) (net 13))
 (segment (start 115.355 102.705) (end 118 100.06) (width 0.35) (layer F.Cu) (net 14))
 (segment (start 111.3 102.705) (end 115.355 102.705) (width 0.35) (layer F.Cu) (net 14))
 (segment (start 121.06 100.06) (end 121.4 100.4) (width 0.35) (layer F.Cu) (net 14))
 (segment (start 118 100.06) (end 121.06 100.06) (width 0.35) (layer F.Cu) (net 14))
 (segment (start 111.3 103.975) (end 115.025 103.975) (width 0.35) (layer F.Cu) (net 15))
 (segment (start 116.4 102.6) (end 118 102.6) (width 0.35) (layer F.Cu) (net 15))
 (segment (start 115.025 103.975) (end 116.4 102.6) (width 0.35) (layer F.Cu) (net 15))
 (segment (start 118 102.6) (end 121.4 102.6) (width 0.35) (layer F.Cu) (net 15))
 (segment (start 121.4 102.6) (end 122.85 104.05) (width 0.35) (layer F.Cu) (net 15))
 (segment (start 122.85 109.25) (end 124.2 110.6) (width 0.35) (layer F.Cu) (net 15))
 (segment (start 122.85 104.05) (end 122.85 109.25) (width 0.35) (layer F.Cu) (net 15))
 (segment (start 117.895 105.245) (end 118 105.14) (width 0.35) (layer F.Cu) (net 16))
 (segment (start 111.3 105.245) (end 117.895 105.245) (width 0.35) (layer F.Cu) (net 16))
 (segment (start 121.34 105.14) (end 121.4 105.2) (width 0.35) (layer F.Cu) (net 16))
 (segment (start 118 105.14) (end 121.34 105.14) (width 0.35) (layer F.Cu) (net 16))
 (segment (start 100.665 105.245) (end 100.6 105.18) (width 0.35) (layer F.Cu) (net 17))
 (segment (start 112.8 109.875) (end 112.8 110.6) (width 0.35) (layer F.Cu) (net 17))
 (segment (start 111.125 108.2) (end 112.8 109.875) (width 0.35) (layer F.Cu) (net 17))
 (segment (start 108.205 108.2) (end 111.125 108.2) (width 0.35) (layer F.Cu) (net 17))
 (segment (start 105.9 105.895) (end 108.205 108.2) (width 0.35) (layer F.Cu) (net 17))
 (segment (start 105.9 105.245) (end 105.9 105.895) (width 0.35) (layer F.Cu) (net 17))
 (segment (start 100.325 105.245) (end 100.22 105.14) (width 0.35) (layer F.Cu) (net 17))
 (segment (start 105.9 105.245) (end 100.325 105.245) (width 0.35) (layer F.Cu) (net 17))
 (segment (start 107.44999 104.42499) (end 107 103.975) (width 0.35) (layer F.Cu) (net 18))
 (segment (start 107.44999 106.227821) (end 107.44999 104.42499) (width 0.35) (layer F.Cu) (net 18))
 (segment (start 116.6 110.6) (end 116.6 109.875) (width 0.35) (layer F.Cu) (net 18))
 (segment (start 116.6 109.875) (end 114.325 107.6) (width 0.35) (layer F.Cu) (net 18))
 (segment (start 114.325 107.6) (end 108.8 107.6) (width 0.35) (layer F.Cu) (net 18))
 (segment (start 108.8 107.6) (end 107.6 106.4) (width 0.35) (layer F.Cu) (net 18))
 (segment (start 107 103.975) (end 105.9 103.975) (width 0.35) (layer F.Cu) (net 18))
 (segment (start 107.6 106.4) (end 107.6 106.377831) (width 0.35) (layer F.Cu) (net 18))
 (segment (start 107.6 106.377831) (end 107.44999 106.227821) (width 0.35) (layer F.Cu) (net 18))
 (segment (start 101.62 104) (end 100.22 102.6) (width 0.35) (layer F.Cu) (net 18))
 (segment (start 104.775 104) (end 101.62 104) (width 0.35) (layer F.Cu) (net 18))
 (segment (start 105.9 103.975) (end 104.8 103.975) (width 0.35) (layer F.Cu) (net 18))
 (segment (start 104.8 103.975) (end 104.775 104) (width 0.35) (layer F.Cu) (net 18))
 (segment (start 102.865 102.705) (end 100.22 100.06) (width 0.35) (layer F.Cu) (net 19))
 (segment (start 105.9 102.705) (end 102.865 102.705) (width 0.35) (layer F.Cu) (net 19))
 (segment (start 104.135 101.435) (end 100.22 97.52) (width 0.35) (layer F.Cu) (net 20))
 (segment (start 105.9 101.435) (end 104.135 101.435) (width 0.35) (layer F.Cu) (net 20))
 (segment (start 99.370001 98.369999) (end 100.22 97.52) (width 0.35) (layer F.Cu) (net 20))
 (segment (start 98.627822 99.112178) (end 99.370001 98.369999) (width 0.35) (layer F.Cu) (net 20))
 (segment (start 98.627822 106.027822) (end 98.627822 99.112178) (width 0.35) (layer F.Cu) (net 20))
 (segment (start 100.2 107.6) (end 98.627822 106.027822) (width 0.35) (layer F.Cu) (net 20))
 (segment (start 106 107.6) (end 100.2 107.6) (width 0.35) (layer F.Cu) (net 20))
 (segment (start 109 110.6) (end 106 107.6) (width 0.35) (layer F.Cu) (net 20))
 (segment (start 105.45 100.365) (end 105.9 100.365) (width 0.35) (layer F.Cu) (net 21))
 (segment (start 104.765 100.165) (end 105.9 100.165) (width 0.35) (layer F.Cu) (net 21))
 (segment (start 102.4 97.8) (end 104.765 100.165) (width 0.35) (layer F.Cu) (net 21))
 (segment (start 102.4 97.16) (end 100.22 94.98) (width 0.35) (layer F.Cu) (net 21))
 (segment (start 102.4 97.8) (end 102.4 97.16) (width 0.35) (layer F.Cu) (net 21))
 (segment (start 99.370001 95.829999) (end 100.22 94.98) (width 0.35) (layer F.Cu) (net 21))
 (segment (start 98.077814 97.122186) (end 99.370001 95.829999) (width 0.35) (layer F.Cu) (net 21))
 (segment (start 98.077814 106.255644) (end 98.077814 97.122186) (width 0.35) (layer F.Cu) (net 21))
 (segment (start 100.02217 108.2) (end 98.077814 106.255644) (width 0.35) (layer F.Cu) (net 21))
 (segment (start 102.8 108.2) (end 100.02217 108.2) (width 0.35) (layer F.Cu) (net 21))
 (segment (start 105.2 110.6) (end 102.8 108.2) (width 0.35) (layer F.Cu) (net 21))
 (segment (start 105.45 99.095) (end 105.9 99.095) (width 0.35) (layer F.Cu) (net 22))
 (segment (start 105.9 98.895) (end 104.695 98.895) (width 0.35) (layer F.Cu) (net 22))
 (segment (start 104.695 98.895) (end 103.2 97.4) (width 0.35) (layer F.Cu) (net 22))
 (segment (start 103.2 95.42) (end 100.22 92.44) (width 0.35) (layer F.Cu) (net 22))
 (segment (start 103.2 97.4) (end 103.2 95.42) (width 0.35) (layer F.Cu) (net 22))
 (segment (start 99.370001 93.289999) (end 100.22 92.44) (width 0.35) (layer F.Cu) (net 22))
 (segment (start 97.527804 95.132196) (end 99.370001 93.289999) (width 0.35) (layer F.Cu) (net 22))
 (segment (start 97.527804 106.727804) (end 97.527804 95.132196) (width 0.35) (layer F.Cu) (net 22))
 (segment (start 101.4 110.6) (end 97.527804 106.727804) (width 0.35) (layer F.Cu) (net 22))
 (segment (start 105.9 97.625) (end 104.825 97.625) (width 0.35) (layer F.Cu) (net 23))
 (segment (start 104.825 97.625) (end 103.8 96.6) (width 0.35) (layer F.Cu) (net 23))
 (segment (start 103.8 93.48) (end 100.22 89.9) (width 0.35) (layer F.Cu) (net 23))
 (segment (start 103.8 96.6) (end 103.8 93.48) (width 0.35) (layer F.Cu) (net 23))
 (segment (start 99.370001 90.749999) (end 100.22 89.9) (width 0.35) (layer F.Cu) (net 23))
 (segment (start 96.977794 93.142206) (end 99.370001 90.749999) (width 0.35) (layer F.Cu) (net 23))
 (segment (start 96.977794 106.955625) (end 96.977794 93.142206) (width 0.35) (layer F.Cu) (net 23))
 (segment (start 97.6 107.577831) (end 96.977794 106.955625) (width 0.35) (layer F.Cu) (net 23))
 (segment (start 97.6 110.6) (end 97.6 107.577831) (width 0.35) (layer F.Cu) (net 23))
 (segment (start 104.4 96) (end 104.4 90) (width 0.35) (layer F.Cu) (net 24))
 (segment (start 104.755 96.355) (end 104.4 96) (width 0.35) (layer F.Cu) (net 24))
 (segment (start 105.9 96.355) (end 104.755 96.355) (width 0.35) (layer F.Cu) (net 24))
 (segment (start 107 96.355) (end 108 97.355) (width 0.35) (layer F.Cu) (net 24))
 (segment (start 105.9 96.355) (end 107 96.355) (width 0.35) (layer F.Cu) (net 24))
 (segment (start 108 97.355) (end 108 106) (width 0.35) (layer F.Cu) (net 24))
 (segment (start 108 106) (end 109 107) (width 0.35) (layer F.Cu) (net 24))
 (segment (start 109 107) (end 114.4 107) (width 0.35) (layer F.Cu) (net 24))
 (segment (start 114.552821 107.04999) (end 116.4 108.89717) (width 0.35) (layer F.Cu) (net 24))
 (segment (start 114.4 107) (end 114.44999 107.04999) (width 0.35) (layer F.Cu) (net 24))
 (segment (start 114.44999 107.04999) (end 114.552821 107.04999) (width 0.35) (layer F.Cu) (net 24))
 (segment (start 118.69717 108.89717) (end 120.4 110.6) (width 0.35) (layer F.Cu) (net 24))
 (segment (start 116.4 108.89717) (end 118.69717 108.89717) (width 0.35) (layer F.Cu) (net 24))
 (segment (start 101.76 87.36) (end 100.22 87.36) (width 0.35) (layer F.Cu) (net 24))
 (segment (start 104.4 90) (end 101.76 87.36) (width 0.35) (layer F.Cu) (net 24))
 (segment (start 115.2 86.5) (end 112.1 89.6) (width 0.35) (layer F.Cu) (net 26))
 (segment (start 115.2 81) (end 115.2 86.5) (width 0.35) (layer F.Cu) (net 26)))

